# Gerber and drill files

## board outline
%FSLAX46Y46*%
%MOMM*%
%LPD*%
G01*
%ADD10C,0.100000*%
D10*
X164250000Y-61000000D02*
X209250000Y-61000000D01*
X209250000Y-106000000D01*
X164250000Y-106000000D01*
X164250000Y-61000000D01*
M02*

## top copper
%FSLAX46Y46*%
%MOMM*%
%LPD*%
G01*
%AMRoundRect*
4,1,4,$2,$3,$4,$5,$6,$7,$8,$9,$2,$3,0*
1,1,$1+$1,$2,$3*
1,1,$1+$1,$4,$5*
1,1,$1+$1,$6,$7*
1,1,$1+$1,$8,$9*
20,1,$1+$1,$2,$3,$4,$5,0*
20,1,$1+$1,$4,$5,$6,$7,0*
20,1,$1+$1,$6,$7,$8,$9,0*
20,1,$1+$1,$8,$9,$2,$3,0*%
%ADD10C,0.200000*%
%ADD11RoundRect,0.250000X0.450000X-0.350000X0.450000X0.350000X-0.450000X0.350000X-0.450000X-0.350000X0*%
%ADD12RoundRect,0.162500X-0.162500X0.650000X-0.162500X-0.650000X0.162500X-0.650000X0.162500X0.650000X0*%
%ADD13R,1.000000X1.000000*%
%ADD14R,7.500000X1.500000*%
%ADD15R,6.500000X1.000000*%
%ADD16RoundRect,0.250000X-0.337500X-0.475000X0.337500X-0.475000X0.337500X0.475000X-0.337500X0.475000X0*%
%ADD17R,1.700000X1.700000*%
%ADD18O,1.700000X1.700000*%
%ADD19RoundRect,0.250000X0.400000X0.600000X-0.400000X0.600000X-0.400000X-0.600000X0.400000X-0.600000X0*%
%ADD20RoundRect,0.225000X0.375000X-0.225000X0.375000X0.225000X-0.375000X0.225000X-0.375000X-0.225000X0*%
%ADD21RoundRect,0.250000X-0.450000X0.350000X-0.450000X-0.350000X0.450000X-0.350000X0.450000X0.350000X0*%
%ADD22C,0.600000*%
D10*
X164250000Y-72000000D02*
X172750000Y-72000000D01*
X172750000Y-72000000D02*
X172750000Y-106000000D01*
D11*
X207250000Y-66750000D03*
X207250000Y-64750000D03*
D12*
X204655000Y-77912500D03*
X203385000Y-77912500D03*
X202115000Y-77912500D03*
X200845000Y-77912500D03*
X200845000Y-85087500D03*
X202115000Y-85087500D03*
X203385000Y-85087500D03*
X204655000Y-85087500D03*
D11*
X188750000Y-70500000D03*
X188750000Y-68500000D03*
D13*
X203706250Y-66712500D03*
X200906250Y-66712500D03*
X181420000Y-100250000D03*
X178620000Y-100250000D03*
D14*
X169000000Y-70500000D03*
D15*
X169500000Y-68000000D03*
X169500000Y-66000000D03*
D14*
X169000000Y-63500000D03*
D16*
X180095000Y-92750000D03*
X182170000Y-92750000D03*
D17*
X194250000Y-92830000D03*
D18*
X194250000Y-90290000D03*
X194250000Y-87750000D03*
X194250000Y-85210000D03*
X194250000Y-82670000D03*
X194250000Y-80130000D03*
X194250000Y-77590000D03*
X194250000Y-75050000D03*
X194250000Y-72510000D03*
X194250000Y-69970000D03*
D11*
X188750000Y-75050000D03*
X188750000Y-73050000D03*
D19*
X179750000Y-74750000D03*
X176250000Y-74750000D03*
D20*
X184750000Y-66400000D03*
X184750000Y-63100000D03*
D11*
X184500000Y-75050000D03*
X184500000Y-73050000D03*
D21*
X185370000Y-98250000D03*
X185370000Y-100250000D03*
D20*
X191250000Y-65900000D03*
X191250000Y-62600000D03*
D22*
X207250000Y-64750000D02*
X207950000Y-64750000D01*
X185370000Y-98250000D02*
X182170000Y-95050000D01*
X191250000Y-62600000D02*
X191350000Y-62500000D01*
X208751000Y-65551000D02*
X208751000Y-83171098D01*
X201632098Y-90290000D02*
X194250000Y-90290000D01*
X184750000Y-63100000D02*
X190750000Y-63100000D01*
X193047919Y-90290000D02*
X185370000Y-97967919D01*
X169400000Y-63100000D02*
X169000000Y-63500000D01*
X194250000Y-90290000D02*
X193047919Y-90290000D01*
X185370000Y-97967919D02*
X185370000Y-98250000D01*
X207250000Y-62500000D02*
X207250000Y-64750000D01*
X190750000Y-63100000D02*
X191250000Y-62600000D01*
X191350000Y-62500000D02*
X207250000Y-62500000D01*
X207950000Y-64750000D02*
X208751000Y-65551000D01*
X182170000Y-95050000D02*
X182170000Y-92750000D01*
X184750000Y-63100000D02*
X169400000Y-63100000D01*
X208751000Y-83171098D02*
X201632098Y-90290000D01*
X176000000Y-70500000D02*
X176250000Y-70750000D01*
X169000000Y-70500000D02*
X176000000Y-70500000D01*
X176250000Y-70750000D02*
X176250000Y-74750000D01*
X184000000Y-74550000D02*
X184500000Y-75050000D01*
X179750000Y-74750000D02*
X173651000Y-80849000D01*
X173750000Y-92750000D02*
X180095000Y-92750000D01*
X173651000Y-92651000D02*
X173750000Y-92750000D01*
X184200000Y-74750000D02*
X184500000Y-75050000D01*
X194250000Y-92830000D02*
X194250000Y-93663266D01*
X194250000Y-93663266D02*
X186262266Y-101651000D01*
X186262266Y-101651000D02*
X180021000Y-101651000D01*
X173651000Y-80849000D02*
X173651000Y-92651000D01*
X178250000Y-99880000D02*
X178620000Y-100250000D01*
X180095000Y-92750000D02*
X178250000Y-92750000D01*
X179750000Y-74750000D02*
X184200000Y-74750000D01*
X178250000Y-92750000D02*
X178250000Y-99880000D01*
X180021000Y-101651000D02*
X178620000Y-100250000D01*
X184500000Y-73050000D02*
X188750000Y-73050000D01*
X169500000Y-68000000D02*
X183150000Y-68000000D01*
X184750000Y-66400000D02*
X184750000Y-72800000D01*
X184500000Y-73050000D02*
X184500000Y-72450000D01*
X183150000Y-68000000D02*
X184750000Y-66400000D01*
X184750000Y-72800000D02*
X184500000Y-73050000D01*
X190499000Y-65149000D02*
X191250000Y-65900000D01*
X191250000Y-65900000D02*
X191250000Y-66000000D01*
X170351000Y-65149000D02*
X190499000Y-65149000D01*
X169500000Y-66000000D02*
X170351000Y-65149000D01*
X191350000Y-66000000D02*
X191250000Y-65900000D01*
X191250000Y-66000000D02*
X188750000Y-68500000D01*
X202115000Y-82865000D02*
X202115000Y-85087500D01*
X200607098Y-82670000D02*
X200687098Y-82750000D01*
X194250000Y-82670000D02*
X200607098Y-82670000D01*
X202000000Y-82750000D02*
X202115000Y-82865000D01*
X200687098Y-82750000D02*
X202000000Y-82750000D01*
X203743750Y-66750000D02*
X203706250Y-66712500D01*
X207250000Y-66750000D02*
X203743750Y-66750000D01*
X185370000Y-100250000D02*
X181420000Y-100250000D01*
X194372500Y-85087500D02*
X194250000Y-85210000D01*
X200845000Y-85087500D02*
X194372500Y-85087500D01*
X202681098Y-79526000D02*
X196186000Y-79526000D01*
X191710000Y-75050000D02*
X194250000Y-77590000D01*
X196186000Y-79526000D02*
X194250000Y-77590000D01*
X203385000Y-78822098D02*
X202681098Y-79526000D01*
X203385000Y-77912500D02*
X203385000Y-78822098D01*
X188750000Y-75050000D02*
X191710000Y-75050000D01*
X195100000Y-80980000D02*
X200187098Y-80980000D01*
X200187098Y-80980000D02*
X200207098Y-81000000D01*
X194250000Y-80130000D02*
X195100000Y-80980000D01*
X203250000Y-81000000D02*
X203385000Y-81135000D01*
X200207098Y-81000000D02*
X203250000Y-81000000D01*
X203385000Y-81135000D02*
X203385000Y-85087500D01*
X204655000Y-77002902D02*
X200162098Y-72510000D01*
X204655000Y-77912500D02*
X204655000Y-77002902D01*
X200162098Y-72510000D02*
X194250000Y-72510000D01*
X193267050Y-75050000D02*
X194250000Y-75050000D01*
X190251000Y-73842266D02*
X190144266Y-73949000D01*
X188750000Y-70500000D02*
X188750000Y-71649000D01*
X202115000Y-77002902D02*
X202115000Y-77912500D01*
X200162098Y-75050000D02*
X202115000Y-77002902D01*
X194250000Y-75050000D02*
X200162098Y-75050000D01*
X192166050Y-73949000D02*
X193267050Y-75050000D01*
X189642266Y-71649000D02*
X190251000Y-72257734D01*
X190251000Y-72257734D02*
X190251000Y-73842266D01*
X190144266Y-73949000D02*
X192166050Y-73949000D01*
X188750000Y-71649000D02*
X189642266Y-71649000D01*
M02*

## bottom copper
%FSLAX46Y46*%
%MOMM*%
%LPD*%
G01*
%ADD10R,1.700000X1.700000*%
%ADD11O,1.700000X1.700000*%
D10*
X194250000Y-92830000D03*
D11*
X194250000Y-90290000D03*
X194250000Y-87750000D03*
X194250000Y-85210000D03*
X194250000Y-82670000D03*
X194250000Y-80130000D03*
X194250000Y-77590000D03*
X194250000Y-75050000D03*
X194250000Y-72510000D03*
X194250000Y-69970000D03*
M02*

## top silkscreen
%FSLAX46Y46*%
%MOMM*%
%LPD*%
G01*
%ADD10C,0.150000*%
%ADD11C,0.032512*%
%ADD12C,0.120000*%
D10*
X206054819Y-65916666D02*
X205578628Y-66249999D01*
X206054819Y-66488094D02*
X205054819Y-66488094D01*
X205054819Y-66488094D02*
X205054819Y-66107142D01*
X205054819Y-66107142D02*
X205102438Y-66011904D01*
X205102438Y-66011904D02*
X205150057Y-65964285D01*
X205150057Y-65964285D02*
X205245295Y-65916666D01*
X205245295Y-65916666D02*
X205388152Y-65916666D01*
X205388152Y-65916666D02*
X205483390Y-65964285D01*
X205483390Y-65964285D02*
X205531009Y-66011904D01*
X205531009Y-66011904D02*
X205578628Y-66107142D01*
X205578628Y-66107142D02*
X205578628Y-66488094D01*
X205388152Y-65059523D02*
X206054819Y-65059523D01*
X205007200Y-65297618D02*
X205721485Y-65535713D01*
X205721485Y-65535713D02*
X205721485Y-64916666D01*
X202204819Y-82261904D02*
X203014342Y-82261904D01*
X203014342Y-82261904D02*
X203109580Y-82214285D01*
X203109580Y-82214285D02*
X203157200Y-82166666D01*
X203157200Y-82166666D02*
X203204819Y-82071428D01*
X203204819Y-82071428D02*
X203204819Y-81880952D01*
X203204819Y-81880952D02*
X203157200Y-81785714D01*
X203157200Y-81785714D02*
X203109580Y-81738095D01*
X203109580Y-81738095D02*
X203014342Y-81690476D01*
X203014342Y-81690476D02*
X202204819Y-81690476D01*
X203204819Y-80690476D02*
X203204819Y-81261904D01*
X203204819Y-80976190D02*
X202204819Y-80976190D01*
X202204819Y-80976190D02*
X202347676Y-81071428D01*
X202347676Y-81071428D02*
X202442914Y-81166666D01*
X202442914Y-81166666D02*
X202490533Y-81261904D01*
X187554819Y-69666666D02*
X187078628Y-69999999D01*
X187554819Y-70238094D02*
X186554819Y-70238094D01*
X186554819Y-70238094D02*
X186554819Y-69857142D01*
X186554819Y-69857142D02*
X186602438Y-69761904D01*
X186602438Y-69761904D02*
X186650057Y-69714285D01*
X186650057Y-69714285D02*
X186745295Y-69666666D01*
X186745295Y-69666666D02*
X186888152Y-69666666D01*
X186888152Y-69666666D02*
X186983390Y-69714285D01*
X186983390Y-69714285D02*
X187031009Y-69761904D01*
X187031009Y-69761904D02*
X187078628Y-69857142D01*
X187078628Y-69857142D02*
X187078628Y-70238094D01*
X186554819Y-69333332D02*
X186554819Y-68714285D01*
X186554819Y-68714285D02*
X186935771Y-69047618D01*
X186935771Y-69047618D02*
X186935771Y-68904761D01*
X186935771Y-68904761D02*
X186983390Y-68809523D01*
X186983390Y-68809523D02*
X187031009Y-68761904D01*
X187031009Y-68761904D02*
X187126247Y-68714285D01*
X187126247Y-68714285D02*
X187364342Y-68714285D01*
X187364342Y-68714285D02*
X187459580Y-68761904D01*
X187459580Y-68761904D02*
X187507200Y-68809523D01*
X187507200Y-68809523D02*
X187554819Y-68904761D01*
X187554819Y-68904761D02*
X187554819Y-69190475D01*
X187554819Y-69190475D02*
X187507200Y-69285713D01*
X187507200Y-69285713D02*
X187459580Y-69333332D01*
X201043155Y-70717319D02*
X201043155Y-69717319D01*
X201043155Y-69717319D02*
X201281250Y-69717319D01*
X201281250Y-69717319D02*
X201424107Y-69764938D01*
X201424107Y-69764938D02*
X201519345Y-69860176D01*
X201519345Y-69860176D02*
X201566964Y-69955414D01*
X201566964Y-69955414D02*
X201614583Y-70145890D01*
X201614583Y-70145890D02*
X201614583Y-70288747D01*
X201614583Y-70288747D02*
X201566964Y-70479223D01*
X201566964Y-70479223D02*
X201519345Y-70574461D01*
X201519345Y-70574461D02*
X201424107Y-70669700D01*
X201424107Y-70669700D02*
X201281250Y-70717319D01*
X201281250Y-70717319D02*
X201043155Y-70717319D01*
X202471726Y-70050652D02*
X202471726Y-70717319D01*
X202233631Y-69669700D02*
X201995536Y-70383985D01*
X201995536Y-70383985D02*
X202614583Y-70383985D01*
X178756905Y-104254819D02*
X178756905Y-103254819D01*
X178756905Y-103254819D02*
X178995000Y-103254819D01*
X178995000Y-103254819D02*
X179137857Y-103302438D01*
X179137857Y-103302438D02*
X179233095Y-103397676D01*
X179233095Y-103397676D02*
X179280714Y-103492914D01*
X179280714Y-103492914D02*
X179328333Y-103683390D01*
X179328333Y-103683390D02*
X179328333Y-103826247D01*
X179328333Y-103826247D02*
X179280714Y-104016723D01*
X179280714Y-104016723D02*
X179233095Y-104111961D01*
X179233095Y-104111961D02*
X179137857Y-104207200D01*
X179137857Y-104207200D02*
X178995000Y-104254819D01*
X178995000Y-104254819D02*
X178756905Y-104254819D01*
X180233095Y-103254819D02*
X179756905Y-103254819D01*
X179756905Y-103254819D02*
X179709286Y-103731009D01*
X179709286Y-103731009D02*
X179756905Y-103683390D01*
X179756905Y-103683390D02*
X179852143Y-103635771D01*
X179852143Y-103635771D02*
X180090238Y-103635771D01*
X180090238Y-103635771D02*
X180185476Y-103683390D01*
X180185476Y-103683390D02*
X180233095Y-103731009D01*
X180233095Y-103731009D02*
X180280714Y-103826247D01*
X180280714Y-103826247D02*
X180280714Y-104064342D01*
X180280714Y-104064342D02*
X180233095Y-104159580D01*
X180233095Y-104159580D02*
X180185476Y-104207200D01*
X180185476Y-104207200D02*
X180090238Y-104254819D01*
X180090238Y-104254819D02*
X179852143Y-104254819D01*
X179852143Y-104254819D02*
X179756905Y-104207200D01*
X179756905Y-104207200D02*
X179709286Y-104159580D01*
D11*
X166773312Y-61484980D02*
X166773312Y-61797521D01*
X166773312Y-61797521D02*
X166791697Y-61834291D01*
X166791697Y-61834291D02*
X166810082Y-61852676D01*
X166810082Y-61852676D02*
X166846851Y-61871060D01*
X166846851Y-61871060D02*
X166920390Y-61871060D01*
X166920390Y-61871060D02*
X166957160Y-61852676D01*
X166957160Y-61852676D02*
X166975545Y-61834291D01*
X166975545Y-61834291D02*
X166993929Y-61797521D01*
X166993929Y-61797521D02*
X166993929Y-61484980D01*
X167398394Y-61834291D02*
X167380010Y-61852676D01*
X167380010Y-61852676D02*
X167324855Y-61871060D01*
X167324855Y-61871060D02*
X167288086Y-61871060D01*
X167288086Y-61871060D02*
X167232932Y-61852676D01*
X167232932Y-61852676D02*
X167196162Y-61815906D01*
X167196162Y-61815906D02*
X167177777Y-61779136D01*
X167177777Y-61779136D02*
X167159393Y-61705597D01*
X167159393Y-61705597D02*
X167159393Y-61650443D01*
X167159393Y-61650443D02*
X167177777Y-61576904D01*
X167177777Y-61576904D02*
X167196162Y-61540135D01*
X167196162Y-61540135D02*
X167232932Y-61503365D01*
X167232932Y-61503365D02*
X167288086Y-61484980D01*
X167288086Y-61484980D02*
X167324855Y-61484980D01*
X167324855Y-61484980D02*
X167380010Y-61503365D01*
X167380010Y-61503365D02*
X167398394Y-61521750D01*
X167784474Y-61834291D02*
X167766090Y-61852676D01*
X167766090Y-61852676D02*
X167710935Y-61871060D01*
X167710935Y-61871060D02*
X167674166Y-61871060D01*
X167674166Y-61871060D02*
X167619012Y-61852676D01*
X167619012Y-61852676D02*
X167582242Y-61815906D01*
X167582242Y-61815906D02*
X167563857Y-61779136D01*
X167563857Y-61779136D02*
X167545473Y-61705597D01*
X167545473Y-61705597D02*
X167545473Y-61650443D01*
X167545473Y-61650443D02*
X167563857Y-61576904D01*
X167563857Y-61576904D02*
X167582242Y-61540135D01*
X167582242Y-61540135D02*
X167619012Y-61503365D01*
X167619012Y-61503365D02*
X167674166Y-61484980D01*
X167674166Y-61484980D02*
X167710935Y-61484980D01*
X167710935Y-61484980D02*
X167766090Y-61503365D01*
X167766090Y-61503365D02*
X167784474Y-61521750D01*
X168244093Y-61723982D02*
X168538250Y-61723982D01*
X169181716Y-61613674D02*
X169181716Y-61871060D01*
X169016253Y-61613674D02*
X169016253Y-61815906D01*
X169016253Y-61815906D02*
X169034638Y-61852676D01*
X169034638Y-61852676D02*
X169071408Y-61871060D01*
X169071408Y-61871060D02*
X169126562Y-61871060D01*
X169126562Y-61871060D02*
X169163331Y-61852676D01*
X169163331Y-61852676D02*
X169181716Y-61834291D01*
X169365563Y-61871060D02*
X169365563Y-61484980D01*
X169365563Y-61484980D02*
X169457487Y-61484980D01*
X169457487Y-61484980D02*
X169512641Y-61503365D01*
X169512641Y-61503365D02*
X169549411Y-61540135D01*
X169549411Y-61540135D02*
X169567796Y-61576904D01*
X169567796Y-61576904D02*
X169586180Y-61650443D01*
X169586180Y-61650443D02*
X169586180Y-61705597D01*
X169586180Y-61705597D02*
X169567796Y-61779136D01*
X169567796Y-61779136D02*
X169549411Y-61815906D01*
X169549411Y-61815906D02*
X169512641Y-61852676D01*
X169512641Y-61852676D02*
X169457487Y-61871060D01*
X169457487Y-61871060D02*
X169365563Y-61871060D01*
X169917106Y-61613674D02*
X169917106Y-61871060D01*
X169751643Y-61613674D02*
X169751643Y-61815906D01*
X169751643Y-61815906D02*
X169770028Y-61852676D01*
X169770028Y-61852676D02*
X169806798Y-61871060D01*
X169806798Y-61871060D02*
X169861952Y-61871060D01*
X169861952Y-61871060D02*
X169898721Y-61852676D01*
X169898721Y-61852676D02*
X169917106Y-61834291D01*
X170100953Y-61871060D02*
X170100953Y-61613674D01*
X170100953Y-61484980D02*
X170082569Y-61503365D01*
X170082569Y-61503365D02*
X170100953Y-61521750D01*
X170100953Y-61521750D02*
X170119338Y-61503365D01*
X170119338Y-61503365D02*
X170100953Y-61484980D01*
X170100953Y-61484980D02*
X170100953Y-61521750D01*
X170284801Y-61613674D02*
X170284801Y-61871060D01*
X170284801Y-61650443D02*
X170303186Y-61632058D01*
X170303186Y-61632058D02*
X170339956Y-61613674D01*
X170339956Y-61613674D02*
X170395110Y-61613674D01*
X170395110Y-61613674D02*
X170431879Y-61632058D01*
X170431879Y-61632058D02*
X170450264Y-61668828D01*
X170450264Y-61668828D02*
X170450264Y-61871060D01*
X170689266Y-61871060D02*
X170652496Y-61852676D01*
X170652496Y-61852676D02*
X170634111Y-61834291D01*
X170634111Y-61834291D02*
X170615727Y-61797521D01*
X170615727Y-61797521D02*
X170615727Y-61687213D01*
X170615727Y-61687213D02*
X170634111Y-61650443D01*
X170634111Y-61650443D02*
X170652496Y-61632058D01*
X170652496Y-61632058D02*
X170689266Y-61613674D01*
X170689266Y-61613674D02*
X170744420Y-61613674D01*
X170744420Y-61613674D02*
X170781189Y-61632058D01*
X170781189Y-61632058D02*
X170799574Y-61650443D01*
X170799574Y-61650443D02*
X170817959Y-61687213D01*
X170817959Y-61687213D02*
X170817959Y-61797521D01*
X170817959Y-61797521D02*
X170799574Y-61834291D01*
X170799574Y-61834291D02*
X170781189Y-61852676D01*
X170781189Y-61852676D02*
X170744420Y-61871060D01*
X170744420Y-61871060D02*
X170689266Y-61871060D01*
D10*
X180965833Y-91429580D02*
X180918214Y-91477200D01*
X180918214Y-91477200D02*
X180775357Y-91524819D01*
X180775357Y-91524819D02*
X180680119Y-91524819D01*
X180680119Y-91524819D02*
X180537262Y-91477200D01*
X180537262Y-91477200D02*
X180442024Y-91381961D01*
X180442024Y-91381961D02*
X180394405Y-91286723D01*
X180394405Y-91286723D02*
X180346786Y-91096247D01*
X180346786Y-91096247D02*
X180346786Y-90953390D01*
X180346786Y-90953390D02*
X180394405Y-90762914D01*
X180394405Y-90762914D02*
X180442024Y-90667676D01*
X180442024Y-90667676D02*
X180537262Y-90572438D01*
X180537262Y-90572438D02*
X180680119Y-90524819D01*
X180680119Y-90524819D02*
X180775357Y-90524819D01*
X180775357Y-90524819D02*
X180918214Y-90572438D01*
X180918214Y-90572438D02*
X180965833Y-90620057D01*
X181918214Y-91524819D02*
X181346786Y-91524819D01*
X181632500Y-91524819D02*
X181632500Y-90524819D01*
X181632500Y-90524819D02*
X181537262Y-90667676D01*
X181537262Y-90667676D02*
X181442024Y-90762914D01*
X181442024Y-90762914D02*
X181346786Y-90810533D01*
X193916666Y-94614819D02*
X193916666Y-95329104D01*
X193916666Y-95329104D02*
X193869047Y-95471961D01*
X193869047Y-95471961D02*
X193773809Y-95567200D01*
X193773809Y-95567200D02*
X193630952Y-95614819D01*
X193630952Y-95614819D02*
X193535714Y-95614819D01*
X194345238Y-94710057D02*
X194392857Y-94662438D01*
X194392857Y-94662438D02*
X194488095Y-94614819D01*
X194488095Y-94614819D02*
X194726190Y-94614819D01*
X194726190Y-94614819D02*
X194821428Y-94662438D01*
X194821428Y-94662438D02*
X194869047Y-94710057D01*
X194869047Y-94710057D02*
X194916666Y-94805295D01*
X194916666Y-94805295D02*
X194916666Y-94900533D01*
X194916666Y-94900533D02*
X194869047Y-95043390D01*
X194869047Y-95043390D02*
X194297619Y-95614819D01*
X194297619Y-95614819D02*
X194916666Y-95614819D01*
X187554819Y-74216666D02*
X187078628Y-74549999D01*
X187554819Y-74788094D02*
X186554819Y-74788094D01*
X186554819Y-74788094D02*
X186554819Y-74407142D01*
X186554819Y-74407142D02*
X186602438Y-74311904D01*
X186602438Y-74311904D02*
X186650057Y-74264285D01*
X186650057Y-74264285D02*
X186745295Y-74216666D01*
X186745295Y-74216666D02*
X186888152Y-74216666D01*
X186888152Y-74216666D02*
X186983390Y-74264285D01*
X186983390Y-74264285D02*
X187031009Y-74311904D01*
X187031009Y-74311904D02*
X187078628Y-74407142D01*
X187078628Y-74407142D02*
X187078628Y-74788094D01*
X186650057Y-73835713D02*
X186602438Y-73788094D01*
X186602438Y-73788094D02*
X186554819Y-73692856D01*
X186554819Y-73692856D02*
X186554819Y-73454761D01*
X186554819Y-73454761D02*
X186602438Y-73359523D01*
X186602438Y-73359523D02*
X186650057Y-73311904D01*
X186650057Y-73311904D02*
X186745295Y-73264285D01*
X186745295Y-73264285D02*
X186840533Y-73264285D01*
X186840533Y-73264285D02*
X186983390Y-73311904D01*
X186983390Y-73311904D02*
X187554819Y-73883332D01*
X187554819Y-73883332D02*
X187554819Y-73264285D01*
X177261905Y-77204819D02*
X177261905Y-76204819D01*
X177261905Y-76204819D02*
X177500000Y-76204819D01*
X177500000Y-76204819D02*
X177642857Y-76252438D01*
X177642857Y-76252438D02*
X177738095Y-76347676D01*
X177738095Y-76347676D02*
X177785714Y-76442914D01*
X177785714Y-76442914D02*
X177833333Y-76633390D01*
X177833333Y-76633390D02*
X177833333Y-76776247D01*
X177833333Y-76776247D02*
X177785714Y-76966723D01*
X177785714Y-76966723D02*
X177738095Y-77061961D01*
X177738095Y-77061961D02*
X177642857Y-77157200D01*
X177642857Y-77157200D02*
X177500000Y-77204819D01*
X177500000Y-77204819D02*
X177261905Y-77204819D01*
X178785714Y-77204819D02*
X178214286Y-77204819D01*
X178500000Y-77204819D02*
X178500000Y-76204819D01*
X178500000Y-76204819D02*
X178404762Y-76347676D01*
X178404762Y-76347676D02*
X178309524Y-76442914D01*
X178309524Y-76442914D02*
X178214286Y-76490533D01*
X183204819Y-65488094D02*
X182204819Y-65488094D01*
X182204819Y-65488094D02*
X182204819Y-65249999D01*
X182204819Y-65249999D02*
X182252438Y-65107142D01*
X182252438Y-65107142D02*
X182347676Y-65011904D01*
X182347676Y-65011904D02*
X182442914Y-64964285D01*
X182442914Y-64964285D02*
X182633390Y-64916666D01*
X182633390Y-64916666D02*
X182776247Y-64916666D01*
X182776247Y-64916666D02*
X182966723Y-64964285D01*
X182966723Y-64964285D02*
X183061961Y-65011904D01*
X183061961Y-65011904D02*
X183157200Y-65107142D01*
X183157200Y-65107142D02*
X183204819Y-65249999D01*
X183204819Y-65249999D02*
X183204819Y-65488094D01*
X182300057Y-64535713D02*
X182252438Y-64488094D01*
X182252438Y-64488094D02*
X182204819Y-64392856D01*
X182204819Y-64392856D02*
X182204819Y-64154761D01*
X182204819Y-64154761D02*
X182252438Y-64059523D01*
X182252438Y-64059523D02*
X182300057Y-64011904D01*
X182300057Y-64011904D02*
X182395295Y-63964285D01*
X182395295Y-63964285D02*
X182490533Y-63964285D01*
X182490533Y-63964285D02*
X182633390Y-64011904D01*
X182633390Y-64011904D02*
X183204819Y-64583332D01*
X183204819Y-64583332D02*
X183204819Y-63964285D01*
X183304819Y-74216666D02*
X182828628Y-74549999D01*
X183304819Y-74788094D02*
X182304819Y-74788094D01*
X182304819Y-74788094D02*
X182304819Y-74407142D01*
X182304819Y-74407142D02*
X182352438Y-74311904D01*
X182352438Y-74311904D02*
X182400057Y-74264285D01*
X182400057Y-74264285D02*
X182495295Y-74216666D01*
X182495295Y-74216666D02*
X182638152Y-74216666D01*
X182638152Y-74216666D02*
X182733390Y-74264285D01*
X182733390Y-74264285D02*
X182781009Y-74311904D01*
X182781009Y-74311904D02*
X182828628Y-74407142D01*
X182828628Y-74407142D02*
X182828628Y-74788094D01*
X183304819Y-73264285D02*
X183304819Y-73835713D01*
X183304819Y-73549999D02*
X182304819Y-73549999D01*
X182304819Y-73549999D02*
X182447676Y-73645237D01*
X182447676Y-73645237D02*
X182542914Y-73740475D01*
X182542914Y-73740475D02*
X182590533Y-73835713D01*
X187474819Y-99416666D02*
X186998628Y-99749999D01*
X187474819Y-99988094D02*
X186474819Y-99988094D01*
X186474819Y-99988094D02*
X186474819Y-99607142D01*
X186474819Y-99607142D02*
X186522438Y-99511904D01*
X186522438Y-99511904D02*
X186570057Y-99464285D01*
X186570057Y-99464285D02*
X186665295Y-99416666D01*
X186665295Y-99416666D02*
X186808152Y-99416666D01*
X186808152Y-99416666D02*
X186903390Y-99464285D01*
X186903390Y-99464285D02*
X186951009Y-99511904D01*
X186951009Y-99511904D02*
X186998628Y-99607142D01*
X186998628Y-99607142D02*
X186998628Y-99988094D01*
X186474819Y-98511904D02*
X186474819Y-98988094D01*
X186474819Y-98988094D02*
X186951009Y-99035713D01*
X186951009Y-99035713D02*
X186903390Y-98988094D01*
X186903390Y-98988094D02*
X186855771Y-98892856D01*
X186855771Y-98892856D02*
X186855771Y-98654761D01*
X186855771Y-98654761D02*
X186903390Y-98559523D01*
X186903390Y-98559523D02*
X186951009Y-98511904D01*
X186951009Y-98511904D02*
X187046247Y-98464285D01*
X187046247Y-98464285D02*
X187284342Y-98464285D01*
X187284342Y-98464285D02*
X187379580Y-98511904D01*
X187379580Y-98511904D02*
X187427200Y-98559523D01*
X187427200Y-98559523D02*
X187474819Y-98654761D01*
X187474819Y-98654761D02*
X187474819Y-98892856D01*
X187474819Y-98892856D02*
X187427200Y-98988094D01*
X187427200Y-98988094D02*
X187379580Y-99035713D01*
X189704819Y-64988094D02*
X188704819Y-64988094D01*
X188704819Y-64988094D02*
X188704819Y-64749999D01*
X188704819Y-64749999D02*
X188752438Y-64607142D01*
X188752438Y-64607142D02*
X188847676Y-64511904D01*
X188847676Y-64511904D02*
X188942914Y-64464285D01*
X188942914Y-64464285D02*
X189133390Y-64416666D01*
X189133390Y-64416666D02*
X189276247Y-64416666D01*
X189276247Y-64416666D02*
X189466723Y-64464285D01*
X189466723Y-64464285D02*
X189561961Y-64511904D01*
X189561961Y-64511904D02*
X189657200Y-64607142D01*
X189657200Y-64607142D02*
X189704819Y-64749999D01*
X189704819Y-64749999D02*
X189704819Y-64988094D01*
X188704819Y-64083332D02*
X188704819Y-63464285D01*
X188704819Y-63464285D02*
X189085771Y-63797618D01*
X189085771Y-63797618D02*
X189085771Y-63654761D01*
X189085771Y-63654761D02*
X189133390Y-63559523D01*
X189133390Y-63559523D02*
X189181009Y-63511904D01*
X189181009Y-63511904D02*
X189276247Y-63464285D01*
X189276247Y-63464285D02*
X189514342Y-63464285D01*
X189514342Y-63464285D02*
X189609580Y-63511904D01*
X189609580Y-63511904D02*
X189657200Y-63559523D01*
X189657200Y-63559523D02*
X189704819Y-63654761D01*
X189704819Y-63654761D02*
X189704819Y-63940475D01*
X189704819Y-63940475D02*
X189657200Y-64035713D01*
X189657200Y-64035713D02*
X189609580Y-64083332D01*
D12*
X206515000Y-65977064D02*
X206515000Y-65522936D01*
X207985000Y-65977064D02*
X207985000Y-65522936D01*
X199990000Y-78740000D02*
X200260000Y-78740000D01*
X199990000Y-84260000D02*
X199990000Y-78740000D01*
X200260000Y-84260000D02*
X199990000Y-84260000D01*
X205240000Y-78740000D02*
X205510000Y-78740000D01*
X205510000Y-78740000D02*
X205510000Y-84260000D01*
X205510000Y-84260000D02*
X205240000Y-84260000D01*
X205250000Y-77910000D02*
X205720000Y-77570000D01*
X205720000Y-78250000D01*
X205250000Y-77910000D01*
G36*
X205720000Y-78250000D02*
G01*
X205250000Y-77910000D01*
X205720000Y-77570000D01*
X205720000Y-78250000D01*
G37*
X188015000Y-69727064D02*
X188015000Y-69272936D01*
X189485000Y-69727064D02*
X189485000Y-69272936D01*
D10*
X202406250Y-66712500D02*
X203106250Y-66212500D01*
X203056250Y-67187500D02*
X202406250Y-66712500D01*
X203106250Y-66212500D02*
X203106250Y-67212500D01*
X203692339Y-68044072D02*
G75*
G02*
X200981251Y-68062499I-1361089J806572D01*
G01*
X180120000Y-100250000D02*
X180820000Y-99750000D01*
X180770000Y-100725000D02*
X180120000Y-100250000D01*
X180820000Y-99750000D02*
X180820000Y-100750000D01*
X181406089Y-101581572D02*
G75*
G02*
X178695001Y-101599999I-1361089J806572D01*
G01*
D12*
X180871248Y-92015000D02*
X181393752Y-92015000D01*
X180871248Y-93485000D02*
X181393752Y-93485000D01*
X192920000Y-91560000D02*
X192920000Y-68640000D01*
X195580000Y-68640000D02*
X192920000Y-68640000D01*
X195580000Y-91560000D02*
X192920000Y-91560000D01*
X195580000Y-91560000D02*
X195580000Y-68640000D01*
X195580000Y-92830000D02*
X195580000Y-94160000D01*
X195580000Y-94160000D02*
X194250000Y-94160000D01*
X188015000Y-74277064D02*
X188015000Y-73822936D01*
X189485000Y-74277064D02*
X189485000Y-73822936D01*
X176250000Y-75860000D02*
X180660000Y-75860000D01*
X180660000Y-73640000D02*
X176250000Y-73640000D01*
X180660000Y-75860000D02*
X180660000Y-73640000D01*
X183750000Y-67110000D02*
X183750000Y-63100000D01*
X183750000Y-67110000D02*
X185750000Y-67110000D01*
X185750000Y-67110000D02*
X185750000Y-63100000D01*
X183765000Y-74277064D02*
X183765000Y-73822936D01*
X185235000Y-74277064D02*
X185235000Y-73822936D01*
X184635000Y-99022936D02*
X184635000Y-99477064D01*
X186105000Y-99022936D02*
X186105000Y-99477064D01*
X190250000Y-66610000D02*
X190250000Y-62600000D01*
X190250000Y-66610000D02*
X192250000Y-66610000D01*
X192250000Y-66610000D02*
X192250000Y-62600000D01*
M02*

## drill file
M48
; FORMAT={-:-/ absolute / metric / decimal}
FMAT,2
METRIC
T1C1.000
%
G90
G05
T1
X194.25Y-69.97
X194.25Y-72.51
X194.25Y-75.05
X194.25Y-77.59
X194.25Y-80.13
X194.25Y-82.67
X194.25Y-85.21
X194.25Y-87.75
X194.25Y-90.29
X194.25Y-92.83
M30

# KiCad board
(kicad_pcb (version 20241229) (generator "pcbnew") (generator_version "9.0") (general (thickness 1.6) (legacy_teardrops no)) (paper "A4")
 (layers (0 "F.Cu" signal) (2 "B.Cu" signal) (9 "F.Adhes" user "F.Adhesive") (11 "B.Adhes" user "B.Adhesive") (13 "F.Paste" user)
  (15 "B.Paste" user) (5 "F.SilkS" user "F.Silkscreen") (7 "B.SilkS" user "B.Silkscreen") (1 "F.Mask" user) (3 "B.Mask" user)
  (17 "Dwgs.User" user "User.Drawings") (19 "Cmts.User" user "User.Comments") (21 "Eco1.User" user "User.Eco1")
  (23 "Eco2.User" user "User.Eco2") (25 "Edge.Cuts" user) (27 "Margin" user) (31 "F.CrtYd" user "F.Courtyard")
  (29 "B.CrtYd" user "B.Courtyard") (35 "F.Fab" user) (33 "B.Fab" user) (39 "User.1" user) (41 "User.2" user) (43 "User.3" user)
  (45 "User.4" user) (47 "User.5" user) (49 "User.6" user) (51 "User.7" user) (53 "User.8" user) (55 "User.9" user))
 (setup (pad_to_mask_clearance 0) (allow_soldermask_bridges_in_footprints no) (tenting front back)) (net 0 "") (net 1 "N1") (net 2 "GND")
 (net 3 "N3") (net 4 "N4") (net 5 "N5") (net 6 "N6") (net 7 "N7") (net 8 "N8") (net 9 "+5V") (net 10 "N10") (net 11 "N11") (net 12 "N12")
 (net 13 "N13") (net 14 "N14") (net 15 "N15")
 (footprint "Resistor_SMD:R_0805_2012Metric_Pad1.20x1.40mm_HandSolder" (layer "F.Cu") (at 207.25 65.75 90)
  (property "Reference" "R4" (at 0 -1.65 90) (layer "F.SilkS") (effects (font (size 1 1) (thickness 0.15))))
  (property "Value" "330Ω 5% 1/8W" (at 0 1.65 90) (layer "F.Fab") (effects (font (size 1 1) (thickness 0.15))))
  (fp_line (start -0.227064 -0.735) (end 0.227064 -0.735) (stroke (width 0.12) (type solid)) (layer "F.SilkS"))
  (fp_line (start -0.227064 0.735) (end 0.227064 0.735) (stroke (width 0.12) (type solid)) (layer "F.SilkS"))
  (pad "1" smd roundrect (at -1 0 90) (size 1.2 1.4) (layers "F.Cu" "F.Mask" "F.Paste") (roundrect_rratio 0.208333) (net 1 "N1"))
  (pad "2" smd roundrect (at 1 0 90) (size 1.2 1.4) (layers "F.Cu" "F.Mask" "F.Paste") (roundrect_rratio 0.208333) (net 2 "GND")))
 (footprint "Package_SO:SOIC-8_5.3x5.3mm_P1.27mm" (layer "F.Cu") (at 202.75 81.5 -90)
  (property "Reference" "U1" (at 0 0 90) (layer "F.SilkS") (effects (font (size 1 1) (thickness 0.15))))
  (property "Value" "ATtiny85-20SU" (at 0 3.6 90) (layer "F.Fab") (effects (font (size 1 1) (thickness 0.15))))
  (fp_line (start -2.76 2.76) (end -2.76 2.49) (stroke (width 0.12) (type solid)) (layer "F.SilkS"))
  (fp_line (start 2.76 2.76) (end -2.76 2.76) (stroke (width 0.12) (type solid)) (layer "F.SilkS"))
  (fp_line (start 2.76 2.49) (end 2.76 2.76) (stroke (width 0.12) (type solid)) (layer "F.SilkS"))
  (fp_line (start -2.76 -2.49) (end -2.76 -2.76) (stroke (width 0.12) (type solid)) (layer "F.SilkS"))
  (fp_line (start -2.76 -2.76) (end 2.76 -2.76) (stroke (width 0.12) (type solid)) (layer "F.SilkS"))
  (fp_line (start 2.76 -2.76) (end 2.76 -2.49) (stroke (width 0.12) (type solid)) (layer "F.SilkS"))
  (fp_poly (pts (xy -3.59 -2.5) (xy -3.93 -2.97) (xy -3.25 -2.97)) (stroke (width 0.12) (type solid)) (fill yes) (layer "F.SilkS"))
  (pad "1" smd roundrect (at -3.5875 -1.905 270) (size 1.625 0.65) (layers "F.Cu" "F.Mask" "F.Paste") (roundrect_rratio 0.25) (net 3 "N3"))
  (pad "2" smd roundrect (at -3.5875 -0.635 270) (size 1.625 0.65) (layers "F.Cu" "F.Mask" "F.Paste") (roundrect_rratio 0.25) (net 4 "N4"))
  (pad "3" smd roundrect (at -3.5875 0.635 270) (size 1.625 0.65) (layers "F.Cu" "F.Mask" "F.Paste") (roundrect_rratio 0.25) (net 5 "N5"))
  (pad "4" smd roundrect (at -3.5875 1.905 270) (size 1.625 0.65) (layers "F.Cu" "F.Mask" "F.Paste") (roundrect_rratio 0.25) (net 2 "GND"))
  (pad "5" smd roundrect (at 3.5875 1.905 270) (size 1.625 0.65) (layers "F.Cu" "F.Mask" "F.Paste") (roundrect_rratio 0.25) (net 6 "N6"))
  (pad "6" smd roundrect (at 3.5875 0.635 270) (size 1.625 0.65) (layers "F.Cu" "F.Mask" "F.Paste") (roundrect_rratio 0.25) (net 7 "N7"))
  (pad "7" smd roundrect (at 3.5875 -0.635 270) (size 1.625 0.65) (layers "F.Cu" "F.Mask" "F.Paste") (roundrect_rratio 0.25) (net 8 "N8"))
  (pad "8" smd roundrect (at 3.5875 -1.905 270) (size 1.625 0.65) (layers "F.Cu" "F.Mask" "F.Paste") (roundrect_rratio 0.25) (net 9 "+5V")))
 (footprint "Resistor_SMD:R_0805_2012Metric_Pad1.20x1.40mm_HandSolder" (layer "F.Cu") (at 188.75 69.5 90)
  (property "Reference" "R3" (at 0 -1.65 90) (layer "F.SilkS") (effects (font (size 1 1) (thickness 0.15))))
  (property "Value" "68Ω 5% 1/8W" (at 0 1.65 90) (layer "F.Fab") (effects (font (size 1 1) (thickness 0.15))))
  (fp_line (start -0.227064 -0.735) (end 0.227064 -0.735) (stroke (width 0.12) (type solid)) (layer "F.SilkS"))
  (fp_line (start -0.227064 0.735) (end 0.227064 0.735) (stroke (width 0.12) (type solid)) (layer "F.SilkS"))
  (pad "1" smd roundrect (at -1 0 90) (size 1.2 1.4) (layers "F.Cu" "F.Mask" "F.Paste") (roundrect_rratio 0.208333) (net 5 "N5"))
  (pad "2" smd roundrect (at 1 0 90) (size 1.2 1.4) (layers "F.Cu" "F.Mask" "F.Paste") (roundrect_rratio 0.208333) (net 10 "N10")))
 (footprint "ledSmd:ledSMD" (layer "F.Cu") (at 201.90625 66.7125 180)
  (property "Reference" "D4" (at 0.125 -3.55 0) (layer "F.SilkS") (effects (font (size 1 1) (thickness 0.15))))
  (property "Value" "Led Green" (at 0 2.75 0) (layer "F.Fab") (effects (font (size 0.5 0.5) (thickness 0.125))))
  (fp_line (start -0.5 0) (end -1.2 0.5) (stroke (width 0.15) (type solid)) (layer "F.SilkS"))
  (fp_line (start -1.15 -0.475) (end -0.5 0) (stroke (width 0.15) (type solid)) (layer "F.SilkS"))
  (fp_line (start -1.2 0.5) (end -1.2 -0.5) (stroke (width 0.15) (type solid)) (layer "F.SilkS"))
  (fp_arc (start -1.786089 -1.331572) (mid -0.435753 -2.107089) (end 0.924999 -1.349999) (stroke (width 0.15) (type solid))
   (layer "F.SilkS"))
  (pad "1" smd rect (at -1.8 0 180) (size 1 1) (layers "F.Cu" "F.Mask" "F.Paste") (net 1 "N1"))
  (pad "2" smd rect (at 1 0 180) (size 1 1) (layers "F.Cu" "F.Mask" "F.Paste") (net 7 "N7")))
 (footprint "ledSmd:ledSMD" (layer "F.Cu") (at 179.62 100.25 180)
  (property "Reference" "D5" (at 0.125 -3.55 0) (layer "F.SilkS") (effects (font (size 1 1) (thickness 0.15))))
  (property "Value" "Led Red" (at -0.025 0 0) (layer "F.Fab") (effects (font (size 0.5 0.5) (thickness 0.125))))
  (fp_line (start -0.5 0) (end -1.2 0.5) (stroke (width 0.15) (type solid)) (layer "F.SilkS"))
  (fp_line (start -1.15 -0.475) (end -0.5 0) (stroke (width 0.15) (type solid)) (layer "F.SilkS"))
  (fp_line (start -1.2 0.5) (end -1.2 -0.5) (stroke (width 0.15) (type solid)) (layer "F.SilkS"))
  (fp_arc (start -1.786089 -1.331572) (mid -0.435753 -2.107089) (end 0.924999 -1.349999) (stroke (width 0.15) (type solid))
   (layer "F.SilkS"))
  (pad "1" smd rect (at -1.8 0 180) (size 1 1) (layers "F.Cu" "F.Mask" "F.Paste") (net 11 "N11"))
  (pad "2" smd rect (at 1 0 180) (size 1 1) (layers "F.Cu" "F.Mask" "F.Paste") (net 9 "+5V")))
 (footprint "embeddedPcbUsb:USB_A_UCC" (layer "F.Cu") (at 169.2 67)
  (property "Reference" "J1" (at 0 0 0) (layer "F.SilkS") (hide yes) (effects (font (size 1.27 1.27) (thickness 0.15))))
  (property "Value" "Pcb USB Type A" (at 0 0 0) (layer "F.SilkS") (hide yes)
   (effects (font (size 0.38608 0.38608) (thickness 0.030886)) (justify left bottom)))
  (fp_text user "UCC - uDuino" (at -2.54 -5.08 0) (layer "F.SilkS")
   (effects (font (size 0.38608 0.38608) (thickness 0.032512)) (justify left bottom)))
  (pad "1" smd rect (at -0.2 3.5) (size 7.5 1.5) (layers "F.Cu" "F.Mask" "F.Paste") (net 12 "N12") (solder_mask_margin 0.1016))
  (pad "2" smd rect (at 0.3 1) (size 6.5 1) (layers "F.Cu" "F.Mask" "F.Paste") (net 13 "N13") (solder_mask_margin 0.1016))
  (pad "3" smd rect (at 0.3 -1) (size 6.5 1) (layers "F.Cu" "F.Mask" "F.Paste") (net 10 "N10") (solder_mask_margin 0.1016))
  (pad "4" smd rect (at -0.2 -3.5) (size 7.5 1.5) (layers "F.Cu" "F.Mask" "F.Paste") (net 2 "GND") (solder_mask_margin 0.1016)))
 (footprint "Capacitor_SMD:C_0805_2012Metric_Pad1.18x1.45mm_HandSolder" (layer "F.Cu") (at 181.1325 92.75)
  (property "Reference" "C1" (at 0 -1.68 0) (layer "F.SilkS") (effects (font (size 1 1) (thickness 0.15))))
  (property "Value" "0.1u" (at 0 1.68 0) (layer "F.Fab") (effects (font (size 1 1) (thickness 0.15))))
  (fp_line (start -0.261252 -0.735) (end 0.261252 -0.735) (stroke (width 0.12) (type solid)) (layer "F.SilkS"))
  (fp_line (start -0.261252 0.735) (end 0.261252 0.735) (stroke (width 0.12) (type solid)) (layer "F.SilkS"))
  (pad "1" smd roundrect (at -1.0375 0) (size 1.175 1.45) (layers "F.Cu" "F.Mask" "F.Paste") (roundrect_rratio 0.212766) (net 9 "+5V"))
  (pad "2" smd roundrect (at 1.0375 0) (size 1.175 1.45) (layers "F.Cu" "F.Mask" "F.Paste") (roundrect_rratio 0.212766) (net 2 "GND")))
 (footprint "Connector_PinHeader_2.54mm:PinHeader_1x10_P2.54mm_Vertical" (layer "F.Cu") (at 194.25 92.83 180)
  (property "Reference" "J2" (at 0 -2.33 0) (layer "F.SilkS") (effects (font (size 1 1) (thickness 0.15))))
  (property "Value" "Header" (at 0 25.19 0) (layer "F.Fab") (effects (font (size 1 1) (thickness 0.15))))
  (fp_line (start 1.33 1.27) (end 1.33 24.19) (stroke (width 0.12) (type solid)) (layer "F.SilkS"))
  (fp_line (start -1.33 24.19) (end 1.33 24.19) (stroke (width 0.12) (type solid)) (layer "F.SilkS"))
  (fp_line (start -1.33 1.27) (end 1.33 1.27) (stroke (width 0.12) (type solid)) (layer "F.SilkS"))
  (fp_line (start -1.33 1.27) (end -1.33 24.19) (stroke (width 0.12) (type solid)) (layer "F.SilkS"))
  (fp_line (start -1.33 0) (end -1.33 -1.33) (stroke (width 0.12) (type solid)) (layer "F.SilkS"))
  (fp_line (start -1.33 -1.33) (end 0 -1.33) (stroke (width 0.12) (type solid)) (layer "F.SilkS"))
  (pad "1" thru_hole rect (at 0 0 180) (size 1.7 1.7) (drill 1) (layers "*.Cu" "*.Mask") (remove_unused_layers no) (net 9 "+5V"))
  (pad "2" thru_hole oval (at 0 2.54 180) (size 1.7 1.7) (drill 1) (layers "*.Cu" "*.Mask") (remove_unused_layers no) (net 2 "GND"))
  (pad "3" thru_hole oval (at 0 5.08 180) (size 1.7 1.7) (drill 1) (layers "*.Cu" "*.Mask") (remove_unused_layers no) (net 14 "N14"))
  (pad "4" thru_hole oval (at 0 7.62 180) (size 1.7 1.7) (drill 1) (layers "*.Cu" "*.Mask") (remove_unused_layers no) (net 6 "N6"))
  (pad "5" thru_hole oval (at 0 10.16 180) (size 1.7 1.7) (drill 1) (layers "*.Cu" "*.Mask") (remove_unused_layers no) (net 7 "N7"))
  (pad "6" thru_hole oval (at 0 12.7 180) (size 1.7 1.7) (drill 1) (layers "*.Cu" "*.Mask") (remove_unused_layers no) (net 8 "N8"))
  (pad "7" thru_hole oval (at 0 15.24 180) (size 1.7 1.7) (drill 1) (layers "*.Cu" "*.Mask") (remove_unused_layers no) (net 4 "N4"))
  (pad "8" thru_hole oval (at 0 17.78 180) (size 1.7 1.7) (drill 1) (layers "*.Cu" "*.Mask") (remove_unused_layers no) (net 5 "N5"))
  (pad "9" thru_hole oval (at 0 20.32 180) (size 1.7 1.7) (drill 1) (layers "*.Cu" "*.Mask") (remove_unused_layers no) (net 3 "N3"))
  (pad "10" thru_hole oval (at 0 22.86 180) (size 1.7 1.7) (drill 1) (layers "*.Cu" "*.Mask") (remove_unused_layers no) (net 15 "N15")))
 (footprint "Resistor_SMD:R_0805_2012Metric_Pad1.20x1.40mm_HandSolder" (layer "F.Cu") (at 188.75 74.05 90)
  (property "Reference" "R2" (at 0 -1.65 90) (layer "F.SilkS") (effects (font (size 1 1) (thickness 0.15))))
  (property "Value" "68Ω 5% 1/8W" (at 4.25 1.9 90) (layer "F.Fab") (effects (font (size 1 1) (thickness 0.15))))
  (fp_line (start -0.227064 -0.735) (end 0.227064 -0.735) (stroke (width 0.12) (type solid)) (layer "F.SilkS"))
  (fp_line (start -0.227064 0.735) (end 0.227064 0.735) (stroke (width 0.12) (type solid)) (layer "F.SilkS"))
  (pad "1" smd roundrect (at -1 0 90) (size 1.2 1.4) (layers "F.Cu" "F.Mask" "F.Paste") (roundrect_rratio 0.208333) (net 4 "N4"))
  (pad "2" smd roundrect (at 1 0 90) (size 1.2 1.4) (layers "F.Cu" "F.Mask" "F.Paste") (roundrect_rratio 0.208333) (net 13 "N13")))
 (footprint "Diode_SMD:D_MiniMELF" (layer "F.Cu") (at 178 74.75 180)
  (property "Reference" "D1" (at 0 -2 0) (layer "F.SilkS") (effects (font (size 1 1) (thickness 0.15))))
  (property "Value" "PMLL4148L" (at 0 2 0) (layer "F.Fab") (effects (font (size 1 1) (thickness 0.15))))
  (fp_line (start 1.75 -1.11) (end -2.66 -1.11) (stroke (width 0.12) (type solid)) (layer "F.SilkS"))
  (fp_line (start -2.66 1.11) (end 1.75 1.11) (stroke (width 0.12) (type solid)) (layer "F.SilkS"))
  (fp_line (start -2.66 -1.11) (end -2.66 1.11) (stroke (width 0.12) (type solid)) (layer "F.SilkS"))
  (pad "1" smd roundrect (at -1.75 0 180) (size 1.3 1.7) (layers "F.Cu" "F.Mask" "F.Paste") (roundrect_rratio 0.1923076923) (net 9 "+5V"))
  (pad "2" smd roundrect (at 1.75 0 180) (size 1.3 1.7) (layers "F.Cu" "F.Mask" "F.Paste") (roundrect_rratio 0.1923076923) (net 12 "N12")))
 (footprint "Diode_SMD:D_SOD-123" (layer "F.Cu") (at 184.75 64.75 90)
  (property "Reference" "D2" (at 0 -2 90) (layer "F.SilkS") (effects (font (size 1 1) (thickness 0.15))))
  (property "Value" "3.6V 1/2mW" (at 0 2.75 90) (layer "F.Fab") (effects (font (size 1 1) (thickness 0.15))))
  (fp_line (start -2.36 -1) (end 1.65 -1) (stroke (width 0.12) (type solid)) (layer "F.SilkS"))
  (fp_line (start -2.36 -1) (end -2.36 1) (stroke (width 0.12) (type solid)) (layer "F.SilkS"))
  (fp_line (start -2.36 1) (end 1.65 1) (stroke (width 0.12) (type solid)) (layer "F.SilkS"))
  (pad "1" smd roundrect (at -1.65 0 90) (size 0.9 1.2) (layers "F.Cu" "F.Mask" "F.Paste") (roundrect_rratio 0.25) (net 13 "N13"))
  (pad "2" smd roundrect (at 1.65 0 90) (size 0.9 1.2) (layers "F.Cu" "F.Mask" "F.Paste") (roundrect_rratio 0.25) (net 2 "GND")))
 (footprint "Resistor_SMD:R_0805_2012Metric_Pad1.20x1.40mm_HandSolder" (layer "F.Cu") (at 184.5 74.05 90)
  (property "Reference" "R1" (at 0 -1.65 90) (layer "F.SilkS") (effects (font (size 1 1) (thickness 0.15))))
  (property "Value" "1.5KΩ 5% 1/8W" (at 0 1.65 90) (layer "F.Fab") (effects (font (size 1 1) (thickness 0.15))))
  (fp_line (start -0.227064 -0.735) (end 0.227064 -0.735) (stroke (width 0.12) (type solid)) (layer "F.SilkS"))
  (fp_line (start -0.227064 0.735) (end 0.227064 0.735) (stroke (width 0.12) (type solid)) (layer "F.SilkS"))
  (pad "1" smd roundrect (at -1 0 90) (size 1.2 1.4) (layers "F.Cu" "F.Mask" "F.Paste") (roundrect_rratio 0.208333) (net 9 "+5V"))
  (pad "2" smd roundrect (at 1 0 90) (size 1.2 1.4) (layers "F.Cu" "F.Mask" "F.Paste") (roundrect_rratio 0.208333) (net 13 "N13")))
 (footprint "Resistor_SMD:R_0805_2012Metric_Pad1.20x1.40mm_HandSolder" (layer "F.Cu") (at 185.37 99.25 -90)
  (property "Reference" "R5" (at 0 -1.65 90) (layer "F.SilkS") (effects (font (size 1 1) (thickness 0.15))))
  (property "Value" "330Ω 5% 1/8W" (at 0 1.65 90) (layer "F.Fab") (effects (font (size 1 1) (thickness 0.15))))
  (fp_line (start -0.227064 0.735) (end 0.227064 0.735) (stroke (width 0.12) (type solid)) (layer "F.SilkS"))
  (fp_line (start -0.227064 -0.735) (end 0.227064 -0.735) (stroke (width 0.12) (type solid)) (layer "F.SilkS"))
  (pad "1" smd roundrect (at -1 0 270) (size 1.2 1.4) (layers "F.Cu" "F.Mask" "F.Paste") (roundrect_rratio 0.208333) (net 2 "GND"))
  (pad "2" smd roundrect (at 1 0 270) (size 1.2 1.4) (layers "F.Cu" "F.Mask" "F.Paste") (roundrect_rratio 0.208333) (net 11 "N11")))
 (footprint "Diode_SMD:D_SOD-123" (layer "F.Cu") (at 191.25 64.25 90)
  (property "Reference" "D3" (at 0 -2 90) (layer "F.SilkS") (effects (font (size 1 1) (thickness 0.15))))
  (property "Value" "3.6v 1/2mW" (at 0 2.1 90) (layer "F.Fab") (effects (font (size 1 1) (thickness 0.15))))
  (fp_line (start -2.36 -1) (end 1.65 -1) (stroke (width 0.12) (type solid)) (layer "F.SilkS"))
  (fp_line (start -2.36 -1) (end -2.36 1) (stroke (width 0.12) (type solid)) (layer "F.SilkS"))
  (fp_line (start -2.36 1) (end 1.65 1) (stroke (width 0.12) (type solid)) (layer "F.SilkS"))
  (pad "1" smd roundrect (at -1.65 0 90) (size 0.9 1.2) (layers "F.Cu" "F.Mask" "F.Paste") (roundrect_rratio 0.25) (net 10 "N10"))
  (pad "2" smd roundrect (at 1.65 0 90) (size 0.9 1.2) (layers "F.Cu" "F.Mask" "F.Paste") (roundrect_rratio 0.25) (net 2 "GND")))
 (gr_line (start 164.25 72) (end 172.75 72) (stroke (width 0.2) (type default)) (layer "F.Cu"))
 (gr_line (start 172.75 72) (end 172.75 106) (stroke (width 0.2) (type default)) (layer "F.Cu"))
 (gr_rect (start 164.25 61) (end 209.25 106) (stroke (width 0.1) (type default)) (fill no) (layer "Edge.Cuts"))
 (segment (start 207.25 64.75) (end 207.95 64.75) (width 0.6) (layer "F.Cu") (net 2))
 (segment (start 185.37 98.25) (end 182.17 95.05) (width 0.6) (layer "F.Cu") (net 2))
 (segment (start 191.25 62.6) (end 191.35 62.5) (width 0.6) (layer "F.Cu") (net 2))
 (segment (start 208.751 65.551) (end 208.751 83.171098) (width 0.6) (layer "F.Cu") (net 2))
 (segment (start 201.632098 90.29) (end 194.25 90.29) (width 0.6) (layer "F.Cu") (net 2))
 (segment (start 184.75 63.1) (end 190.75 63.1) (width 0.6) (layer "F.Cu") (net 2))
 (segment (start 193.047919 90.29) (end 185.37 97.967919) (width 0.6) (layer "F.Cu") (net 2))
 (segment (start 169.4 63.1) (end 169 63.5) (width 0.6) (layer "F.Cu") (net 2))
 (segment (start 194.25 90.29) (end 193.047919 90.29) (width 0.6) (layer "F.Cu") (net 2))
 (segment (start 185.37 97.967919) (end 185.37 98.25) (width 0.6) (layer "F.Cu") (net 2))
 (segment (start 207.25 62.5) (end 207.25 64.75) (width 0.6) (layer "F.Cu") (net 2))
 (segment (start 190.75 63.1) (end 191.25 62.6) (width 0.6) (layer "F.Cu") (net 2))
 (segment (start 191.35 62.5) (end 207.25 62.5) (width 0.6) (layer "F.Cu") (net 2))
 (segment (start 207.95 64.75) (end 208.751 65.551) (width 0.6) (layer "F.Cu") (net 2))
 (segment (start 182.17 95.05) (end 182.17 92.75) (width 0.6) (layer "F.Cu") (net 2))
 (segment (start 184.75 63.1) (end 169.4 63.1) (width 0.6) (layer "F.Cu") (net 2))
 (segment (start 208.751 83.171098) (end 201.632098 90.29) (width 0.6) (layer "F.Cu") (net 2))
 (segment (start 176 70.5) (end 176.25 70.75) (width 0.6) (layer "F.Cu") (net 12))
 (segment (start 169 70.5) (end 176 70.5) (width 0.6) (layer "F.Cu") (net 12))
 (segment (start 176.25 70.75) (end 176.25 74.75) (width 0.6) (layer "F.Cu") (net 12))
 (segment (start 184 74.55) (end 184.5 75.05) (width 0.6) (layer "F.Cu") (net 9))
 (segment (start 179.75 74.75) (end 173.651 80.849) (width 0.6) (layer "F.Cu") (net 9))
 (segment (start 173.75 92.75) (end 180.095 92.75) (width 0.6) (layer "F.Cu") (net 9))
 (segment (start 173.651 92.651) (end 173.75 92.75) (width 0.6) (layer "F.Cu") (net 9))
 (segment (start 184.2 74.75) (end 184.5 75.05) (width 0.6) (layer "F.Cu") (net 9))
 (segment (start 194.25 92.83) (end 194.25 93.663266) (width 0.6) (layer "F.Cu") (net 9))
 (segment (start 194.25 93.663266) (end 186.262266 101.651) (width 0.6) (layer "F.Cu") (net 9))
 (segment (start 186.262266 101.651) (end 180.021 101.651) (width 0.6) (layer "F.Cu") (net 9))
 (segment (start 173.651 80.849) (end 173.651 92.651) (width 0.6) (layer "F.Cu") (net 9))
 (segment (start 178.25 99.88) (end 178.62 100.25) (width 0.6) (layer "F.Cu") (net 9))
 (segment (start 180.095 92.75) (end 178.25 92.75) (width 0.6) (layer "F.Cu") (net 9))
 (segment (start 179.75 74.75) (end 184.2 74.75) (width 0.6) (layer "F.Cu") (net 9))
 (segment (start 178.25 92.75) (end 178.25 99.88) (width 0.6) (layer "F.Cu") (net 9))
 (segment (start 180.021 101.651) (end 178.62 100.25) (width 0.6) (layer "F.Cu") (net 9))
 (segment (start 184.5 73.05) (end 188.75 73.05) (width 0.6) (layer "F.Cu") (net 13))
 (segment (start 169.5 68) (end 183.15 68) (width 0.6) (layer "F.Cu") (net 13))
 (segment (start 184.75 66.4) (end 184.75 72.8) (width 0.6) (layer "F.Cu") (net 13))
 (segment (start 184.5 73.05) (end 184.5 72.45) (width 0.6) (layer "F.Cu") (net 13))
 (segment (start 183.15 68) (end 184.75 66.4) (width 0.6) (layer "F.Cu") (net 13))
 (segment (start 184.75 72.8) (end 184.5 73.05) (width 0.6) (layer "F.Cu") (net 13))
 (segment (start 190.499 65.149) (end 191.25 65.9) (width 0.6) (layer "F.Cu") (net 10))
 (segment (start 191.25 65.9) (end 191.25 66) (width 0.6) (layer "F.Cu") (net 10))
 (segment (start 170.351 65.149) (end 190.499 65.149) (width 0.6) (layer "F.Cu") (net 10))
 (segment (start 169.5 66) (end 170.351 65.149) (width 0.6) (layer "F.Cu") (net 10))
 (segment (start 191.35 66) (end 191.25 65.9) (width 0.6) (layer "F.Cu") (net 10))
 (segment (start 191.25 66) (end 188.75 68.5) (width 0.6) (layer "F.Cu") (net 10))
 (segment (start 202.115 82.865) (end 202.115 85.0875) (width 0.6) (layer "F.Cu") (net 7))
 (segment (start 200.607098 82.67) (end 200.687098 82.75) (width 0.6) (layer "F.Cu") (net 7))
 (segment (start 194.25 82.67) (end 200.607098 82.67) (width 0.6) (layer "F.Cu") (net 7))
 (segment (start 202 82.75) (end 202.115 82.865) (width 0.6) (layer "F.Cu") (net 7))
 (segment (start 200.687098 82.75) (end 202 82.75) (width 0.6) (layer "F.Cu") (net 7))
 (segment (start 203.74375 66.75) (end 203.70625 66.7125) (width 0.6) (layer "F.Cu") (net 1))
 (segment (start 207.25 66.75) (end 203.74375 66.75) (width 0.6) (layer "F.Cu") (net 1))
 (segment (start 185.37 100.25) (end 181.42 100.25) (width 0.6) (layer "F.Cu") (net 11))
 (segment (start 194.3725 85.0875) (end 194.25 85.21) (width 0.6) (layer "F.Cu") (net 6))
 (segment (start 200.845 85.0875) (end 194.3725 85.0875) (width 0.6) (layer "F.Cu") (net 6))
 (segment (start 202.681098 79.526) (end 196.186 79.526) (width 0.6) (layer "F.Cu") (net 4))
 (segment (start 191.71 75.05) (end 194.25 77.59) (width 0.6) (layer "F.Cu") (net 4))
 (segment (start 196.186 79.526) (end 194.25 77.59) (width 0.6) (layer "F.Cu") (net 4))
 (segment (start 203.385 78.822098) (end 202.681098 79.526) (width 0.6) (layer "F.Cu") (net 4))
 (segment (start 203.385 77.9125) (end 203.385 78.822098) (width 0.6) (layer "F.Cu") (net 4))
 (segment (start 188.75 75.05) (end 191.71 75.05) (width 0.6) (layer "F.Cu") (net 4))
 (segment (start 195.1 80.98) (end 200.187098 80.98) (width 0.6) (layer "F.Cu") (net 8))
 (segment (start 200.187098 80.98) (end 200.207098 81) (width 0.6) (layer "F.Cu") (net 8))
 (segment (start 194.25 80.13) (end 195.1 80.98) (width 0.6) (layer "F.Cu") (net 8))
 (segment (start 203.25 81) (end 203.385 81.135) (width 0.6) (layer "F.Cu") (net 8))
 (segment (start 200.207098 81) (end 203.25 81) (width 0.6) (layer "F.Cu") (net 8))
 (segment (start 203.385 81.135) (end 203.385 85.0875) (width 0.6) (layer "F.Cu") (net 8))
 (segment (start 204.655 77.002902) (end 200.162098 72.51) (width 0.6) (layer "F.Cu") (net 3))
 (segment (start 204.655 77.9125) (end 204.655 77.002902) (width 0.6) (layer "F.Cu") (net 3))
 (segment (start 200.162098 72.51) (end 194.25 72.51) (width 0.6) (layer "F.Cu") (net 3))
 (segment (start 193.26705 75.05) (end 194.25 75.05) (width 0.6) (layer "F.Cu") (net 5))
 (segment (start 190.251 73.842266) (end 190.144266 73.949) (width 0.6) (layer "F.Cu") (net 5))
 (segment (start 188.75 70.5) (end 188.75 71.649) (width 0.6) (layer "F.Cu") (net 5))
 (segment (start 202.115 77.002902) (end 202.115 77.9125) (width 0.6) (layer "F.Cu") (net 5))
 (segment (start 200.162098 75.05) (end 202.115 77.002902) (width 0.6) (layer "F.Cu") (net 5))
 (segment (start 194.25 75.05) (end 200.162098 75.05) (width 0.6) (layer "F.Cu") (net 5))
 (segment (start 192.16605 73.949) (end 193.26705 75.05) (width 0.6) (layer "F.Cu") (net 5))
 (segment (start 189.642266 71.649) (end 190.251 72.257734) (width 0.6) (layer "F.Cu") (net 5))
 (segment (start 190.251 72.257734) (end 190.251 73.842266) (width 0.6) (layer "F.Cu") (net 5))
 (segment (start 190.144266 73.949) (end 192.16605 73.949) (width 0.6) (layer "F.Cu") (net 5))
 (segment (start 188.75 71.649) (end 189.642266 71.649) (width 0.6) (layer "F.Cu") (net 5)))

